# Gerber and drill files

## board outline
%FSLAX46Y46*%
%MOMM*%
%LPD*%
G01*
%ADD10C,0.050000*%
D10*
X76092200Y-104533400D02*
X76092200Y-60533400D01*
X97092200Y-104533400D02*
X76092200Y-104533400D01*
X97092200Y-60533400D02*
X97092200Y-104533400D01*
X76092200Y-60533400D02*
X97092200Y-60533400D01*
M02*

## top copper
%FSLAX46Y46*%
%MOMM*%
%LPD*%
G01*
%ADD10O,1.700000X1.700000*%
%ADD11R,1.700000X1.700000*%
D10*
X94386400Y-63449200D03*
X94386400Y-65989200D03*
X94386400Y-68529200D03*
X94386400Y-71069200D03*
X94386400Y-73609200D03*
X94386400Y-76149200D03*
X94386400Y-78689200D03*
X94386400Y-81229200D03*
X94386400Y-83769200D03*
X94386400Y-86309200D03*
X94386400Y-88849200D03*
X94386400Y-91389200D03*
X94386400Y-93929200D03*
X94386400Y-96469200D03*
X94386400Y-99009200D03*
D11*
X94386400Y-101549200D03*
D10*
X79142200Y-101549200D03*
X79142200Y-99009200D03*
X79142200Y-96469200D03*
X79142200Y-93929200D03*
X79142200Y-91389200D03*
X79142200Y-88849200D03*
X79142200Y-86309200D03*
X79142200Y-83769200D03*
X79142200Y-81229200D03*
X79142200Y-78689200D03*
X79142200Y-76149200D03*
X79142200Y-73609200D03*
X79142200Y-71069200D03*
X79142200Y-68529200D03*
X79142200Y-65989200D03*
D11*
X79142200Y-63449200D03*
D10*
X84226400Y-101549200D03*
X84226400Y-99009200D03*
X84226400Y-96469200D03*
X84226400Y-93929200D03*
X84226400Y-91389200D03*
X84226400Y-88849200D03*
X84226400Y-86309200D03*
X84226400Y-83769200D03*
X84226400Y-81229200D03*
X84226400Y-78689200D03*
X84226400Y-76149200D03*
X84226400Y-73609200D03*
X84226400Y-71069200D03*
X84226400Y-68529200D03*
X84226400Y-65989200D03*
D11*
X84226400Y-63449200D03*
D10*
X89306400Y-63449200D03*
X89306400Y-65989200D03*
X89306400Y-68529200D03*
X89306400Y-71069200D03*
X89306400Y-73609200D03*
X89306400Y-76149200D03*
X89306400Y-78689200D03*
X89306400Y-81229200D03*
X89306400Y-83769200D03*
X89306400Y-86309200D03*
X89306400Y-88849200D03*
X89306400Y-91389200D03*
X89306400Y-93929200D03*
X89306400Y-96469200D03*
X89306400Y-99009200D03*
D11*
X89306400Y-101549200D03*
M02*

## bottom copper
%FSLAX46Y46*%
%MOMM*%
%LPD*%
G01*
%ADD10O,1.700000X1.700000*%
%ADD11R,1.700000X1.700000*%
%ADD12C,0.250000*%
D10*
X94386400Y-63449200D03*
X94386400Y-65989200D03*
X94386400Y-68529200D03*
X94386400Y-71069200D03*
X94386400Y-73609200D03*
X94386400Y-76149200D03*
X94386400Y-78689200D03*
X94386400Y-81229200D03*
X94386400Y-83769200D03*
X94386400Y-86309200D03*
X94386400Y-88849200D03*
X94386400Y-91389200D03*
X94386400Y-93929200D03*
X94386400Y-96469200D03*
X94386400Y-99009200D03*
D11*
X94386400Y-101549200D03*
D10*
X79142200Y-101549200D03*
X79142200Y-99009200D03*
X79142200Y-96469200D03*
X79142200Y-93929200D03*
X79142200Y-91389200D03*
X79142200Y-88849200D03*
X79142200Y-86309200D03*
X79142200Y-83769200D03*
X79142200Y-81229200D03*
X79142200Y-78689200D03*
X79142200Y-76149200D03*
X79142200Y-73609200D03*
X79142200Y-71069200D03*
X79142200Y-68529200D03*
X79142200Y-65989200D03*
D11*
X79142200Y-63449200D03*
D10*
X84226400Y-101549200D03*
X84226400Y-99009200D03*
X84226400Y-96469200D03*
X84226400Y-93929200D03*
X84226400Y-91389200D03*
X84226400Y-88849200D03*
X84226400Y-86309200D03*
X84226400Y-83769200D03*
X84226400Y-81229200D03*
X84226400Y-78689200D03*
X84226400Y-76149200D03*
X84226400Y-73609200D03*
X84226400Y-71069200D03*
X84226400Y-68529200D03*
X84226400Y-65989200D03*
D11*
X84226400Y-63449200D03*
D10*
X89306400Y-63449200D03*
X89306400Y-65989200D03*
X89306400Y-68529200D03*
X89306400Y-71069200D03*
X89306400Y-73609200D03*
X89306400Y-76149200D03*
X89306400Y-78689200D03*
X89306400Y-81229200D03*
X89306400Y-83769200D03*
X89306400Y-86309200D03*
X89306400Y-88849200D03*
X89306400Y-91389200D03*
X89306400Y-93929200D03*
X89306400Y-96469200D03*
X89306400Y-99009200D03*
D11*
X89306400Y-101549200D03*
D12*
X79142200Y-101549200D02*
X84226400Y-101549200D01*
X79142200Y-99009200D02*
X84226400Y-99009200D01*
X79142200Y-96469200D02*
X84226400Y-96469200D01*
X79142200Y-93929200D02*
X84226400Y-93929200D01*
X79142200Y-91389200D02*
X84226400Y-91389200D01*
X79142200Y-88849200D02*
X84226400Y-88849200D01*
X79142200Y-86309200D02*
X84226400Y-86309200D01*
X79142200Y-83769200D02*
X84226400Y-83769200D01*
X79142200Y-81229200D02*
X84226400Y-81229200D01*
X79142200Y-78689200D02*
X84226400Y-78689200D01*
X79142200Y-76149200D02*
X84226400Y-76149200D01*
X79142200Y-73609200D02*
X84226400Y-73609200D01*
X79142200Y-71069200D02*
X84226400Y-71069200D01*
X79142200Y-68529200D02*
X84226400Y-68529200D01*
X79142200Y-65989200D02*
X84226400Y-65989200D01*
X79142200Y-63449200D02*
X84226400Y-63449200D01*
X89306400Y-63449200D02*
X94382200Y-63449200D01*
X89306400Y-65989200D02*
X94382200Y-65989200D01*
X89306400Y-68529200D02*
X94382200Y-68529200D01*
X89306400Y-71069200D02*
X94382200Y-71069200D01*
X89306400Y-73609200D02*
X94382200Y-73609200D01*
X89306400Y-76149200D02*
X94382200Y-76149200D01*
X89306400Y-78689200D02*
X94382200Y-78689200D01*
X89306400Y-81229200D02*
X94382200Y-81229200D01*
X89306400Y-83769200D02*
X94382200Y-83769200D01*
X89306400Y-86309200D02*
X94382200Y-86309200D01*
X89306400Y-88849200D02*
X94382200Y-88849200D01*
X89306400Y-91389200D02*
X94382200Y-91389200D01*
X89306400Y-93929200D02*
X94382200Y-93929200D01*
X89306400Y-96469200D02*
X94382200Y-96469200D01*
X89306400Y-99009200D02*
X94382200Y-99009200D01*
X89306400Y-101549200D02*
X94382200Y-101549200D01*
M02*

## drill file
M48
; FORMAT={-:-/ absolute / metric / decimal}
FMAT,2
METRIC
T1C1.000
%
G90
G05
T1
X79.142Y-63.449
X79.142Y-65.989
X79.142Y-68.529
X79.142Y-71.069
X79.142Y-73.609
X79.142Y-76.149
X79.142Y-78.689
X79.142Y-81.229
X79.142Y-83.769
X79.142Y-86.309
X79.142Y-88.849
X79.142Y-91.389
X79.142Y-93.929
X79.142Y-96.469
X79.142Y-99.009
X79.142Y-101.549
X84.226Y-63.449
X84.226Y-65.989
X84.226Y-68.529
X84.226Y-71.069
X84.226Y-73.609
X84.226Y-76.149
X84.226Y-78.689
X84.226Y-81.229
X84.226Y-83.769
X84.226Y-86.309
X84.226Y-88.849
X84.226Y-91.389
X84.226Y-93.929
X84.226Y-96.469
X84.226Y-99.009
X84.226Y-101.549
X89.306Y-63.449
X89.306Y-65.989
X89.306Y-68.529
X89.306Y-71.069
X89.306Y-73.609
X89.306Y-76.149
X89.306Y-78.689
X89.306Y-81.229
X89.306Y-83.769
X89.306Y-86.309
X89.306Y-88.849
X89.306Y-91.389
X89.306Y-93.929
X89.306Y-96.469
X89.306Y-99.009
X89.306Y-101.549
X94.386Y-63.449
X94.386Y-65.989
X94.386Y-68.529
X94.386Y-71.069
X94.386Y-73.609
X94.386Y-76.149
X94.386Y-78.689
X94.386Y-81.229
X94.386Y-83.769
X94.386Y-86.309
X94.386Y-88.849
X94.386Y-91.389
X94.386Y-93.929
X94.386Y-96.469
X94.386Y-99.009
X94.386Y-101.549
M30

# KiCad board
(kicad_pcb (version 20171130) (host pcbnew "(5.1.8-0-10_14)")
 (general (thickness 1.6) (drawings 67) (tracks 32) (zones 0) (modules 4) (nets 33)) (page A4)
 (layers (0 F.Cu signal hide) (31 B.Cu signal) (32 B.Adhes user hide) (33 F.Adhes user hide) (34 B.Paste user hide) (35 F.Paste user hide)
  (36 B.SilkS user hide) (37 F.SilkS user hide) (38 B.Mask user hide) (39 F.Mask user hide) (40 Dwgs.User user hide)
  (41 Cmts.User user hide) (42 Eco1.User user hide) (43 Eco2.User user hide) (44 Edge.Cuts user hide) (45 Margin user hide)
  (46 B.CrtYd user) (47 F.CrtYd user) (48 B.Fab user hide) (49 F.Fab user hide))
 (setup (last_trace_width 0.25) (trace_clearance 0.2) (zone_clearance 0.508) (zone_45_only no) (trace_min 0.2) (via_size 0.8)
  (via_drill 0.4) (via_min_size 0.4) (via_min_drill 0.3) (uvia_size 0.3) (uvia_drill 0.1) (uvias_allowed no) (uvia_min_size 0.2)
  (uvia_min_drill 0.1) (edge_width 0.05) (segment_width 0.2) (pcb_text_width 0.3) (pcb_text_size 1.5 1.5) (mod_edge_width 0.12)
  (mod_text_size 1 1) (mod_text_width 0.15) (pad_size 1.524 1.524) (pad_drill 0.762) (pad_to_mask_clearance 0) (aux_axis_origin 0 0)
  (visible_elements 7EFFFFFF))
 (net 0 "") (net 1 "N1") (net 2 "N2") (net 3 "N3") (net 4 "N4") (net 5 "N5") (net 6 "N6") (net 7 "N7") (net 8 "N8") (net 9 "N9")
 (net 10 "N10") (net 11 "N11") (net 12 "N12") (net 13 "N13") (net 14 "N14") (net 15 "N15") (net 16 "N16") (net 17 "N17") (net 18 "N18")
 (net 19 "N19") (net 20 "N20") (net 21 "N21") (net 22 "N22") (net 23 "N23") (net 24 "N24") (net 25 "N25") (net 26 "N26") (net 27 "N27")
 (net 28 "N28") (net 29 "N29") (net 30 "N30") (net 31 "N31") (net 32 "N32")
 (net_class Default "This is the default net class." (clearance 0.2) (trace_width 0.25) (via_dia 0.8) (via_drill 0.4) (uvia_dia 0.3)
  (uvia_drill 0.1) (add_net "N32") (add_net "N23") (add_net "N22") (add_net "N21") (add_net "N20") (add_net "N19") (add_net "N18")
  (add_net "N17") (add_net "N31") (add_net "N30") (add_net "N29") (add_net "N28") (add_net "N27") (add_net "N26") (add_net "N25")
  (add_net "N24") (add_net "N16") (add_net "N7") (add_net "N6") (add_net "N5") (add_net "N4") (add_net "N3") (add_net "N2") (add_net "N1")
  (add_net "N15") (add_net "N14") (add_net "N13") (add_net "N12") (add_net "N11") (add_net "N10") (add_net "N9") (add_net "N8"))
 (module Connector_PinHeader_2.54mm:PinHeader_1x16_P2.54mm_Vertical (layer F.Cu) (at 94.3864 101.5492 180)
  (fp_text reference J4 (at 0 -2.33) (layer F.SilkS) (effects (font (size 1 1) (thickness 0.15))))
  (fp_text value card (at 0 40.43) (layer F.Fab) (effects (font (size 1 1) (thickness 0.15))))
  (pad 16 thru_hole oval (at 0 38.1 180) (size 1.7 1.7) (drill 1) (layers *.Cu *.Mask) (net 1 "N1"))
  (pad 15 thru_hole oval (at 0 35.56 180) (size 1.7 1.7) (drill 1) (layers *.Cu *.Mask) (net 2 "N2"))
  (pad 14 thru_hole oval (at 0 33.02 180) (size 1.7 1.7) (drill 1) (layers *.Cu *.Mask) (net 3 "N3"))
  (pad 13 thru_hole oval (at 0 30.48 180) (size 1.7 1.7) (drill 1) (layers *.Cu *.Mask) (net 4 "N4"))
  (pad 12 thru_hole oval (at 0 27.94 180) (size 1.7 1.7) (drill 1) (layers *.Cu *.Mask) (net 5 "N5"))
  (pad 11 thru_hole oval (at 0 25.4 180) (size 1.7 1.7) (drill 1) (layers *.Cu *.Mask) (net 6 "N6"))
  (pad 10 thru_hole oval (at 0 22.86 180) (size 1.7 1.7) (drill 1) (layers *.Cu *.Mask) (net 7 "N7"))
  (pad 9 thru_hole oval (at 0 20.32 180) (size 1.7 1.7) (drill 1) (layers *.Cu *.Mask) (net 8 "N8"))
  (pad 8 thru_hole oval (at 0 17.78 180) (size 1.7 1.7) (drill 1) (layers *.Cu *.Mask) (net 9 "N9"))
  (pad 7 thru_hole oval (at 0 15.24 180) (size 1.7 1.7) (drill 1) (layers *.Cu *.Mask) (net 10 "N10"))
  (pad 6 thru_hole oval (at 0 12.7 180) (size 1.7 1.7) (drill 1) (layers *.Cu *.Mask) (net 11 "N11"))
  (pad 5 thru_hole oval (at 0 10.16 180) (size 1.7 1.7) (drill 1) (layers *.Cu *.Mask) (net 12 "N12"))
  (pad 4 thru_hole oval (at 0 7.62 180) (size 1.7 1.7) (drill 1) (layers *.Cu *.Mask) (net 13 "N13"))
  (pad 3 thru_hole oval (at 0 5.08 180) (size 1.7 1.7) (drill 1) (layers *.Cu *.Mask) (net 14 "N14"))
  (pad 2 thru_hole oval (at 0 2.54 180) (size 1.7 1.7) (drill 1) (layers *.Cu *.Mask) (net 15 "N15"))
  (pad 1 thru_hole rect (at 0 0 180) (size 1.7 1.7) (drill 1) (layers *.Cu *.Mask) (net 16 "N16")))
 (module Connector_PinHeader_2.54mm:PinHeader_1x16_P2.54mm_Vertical (layer F.Cu) (at 79.1422 63.4492)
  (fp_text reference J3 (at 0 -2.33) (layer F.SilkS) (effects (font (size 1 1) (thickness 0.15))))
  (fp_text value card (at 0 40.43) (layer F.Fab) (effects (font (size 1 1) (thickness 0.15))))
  (pad 16 thru_hole oval (at 0 38.1) (size 1.7 1.7) (drill 1) (layers *.Cu *.Mask) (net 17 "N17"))
  (pad 15 thru_hole oval (at 0 35.56) (size 1.7 1.7) (drill 1) (layers *.Cu *.Mask) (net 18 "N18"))
  (pad 14 thru_hole oval (at 0 33.02) (size 1.7 1.7) (drill 1) (layers *.Cu *.Mask) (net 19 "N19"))
  (pad 13 thru_hole oval (at 0 30.48) (size 1.7 1.7) (drill 1) (layers *.Cu *.Mask) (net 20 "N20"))
  (pad 12 thru_hole oval (at 0 27.94) (size 1.7 1.7) (drill 1) (layers *.Cu *.Mask) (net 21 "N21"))
  (pad 11 thru_hole oval (at 0 25.4) (size 1.7 1.7) (drill 1) (layers *.Cu *.Mask) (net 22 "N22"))
  (pad 10 thru_hole oval (at 0 22.86) (size 1.7 1.7) (drill 1) (layers *.Cu *.Mask) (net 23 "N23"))
  (pad 9 thru_hole oval (at 0 20.32) (size 1.7 1.7) (drill 1) (layers *.Cu *.Mask) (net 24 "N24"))
  (pad 8 thru_hole oval (at 0 17.78) (size 1.7 1.7) (drill 1) (layers *.Cu *.Mask) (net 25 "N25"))
  (pad 7 thru_hole oval (at 0 15.24) (size 1.7 1.7) (drill 1) (layers *.Cu *.Mask) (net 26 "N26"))
  (pad 6 thru_hole oval (at 0 12.7) (size 1.7 1.7) (drill 1) (layers *.Cu *.Mask) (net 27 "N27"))
  (pad 5 thru_hole oval (at 0 10.16) (size 1.7 1.7) (drill 1) (layers *.Cu *.Mask) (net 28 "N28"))
  (pad 4 thru_hole oval (at 0 7.62) (size 1.7 1.7) (drill 1) (layers *.Cu *.Mask) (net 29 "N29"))
  (pad 3 thru_hole oval (at 0 5.08) (size 1.7 1.7) (drill 1) (layers *.Cu *.Mask) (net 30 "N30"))
  (pad 2 thru_hole oval (at 0 2.54) (size 1.7 1.7) (drill 1) (layers *.Cu *.Mask) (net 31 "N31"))
  (pad 1 thru_hole rect (at 0 0) (size 1.7 1.7) (drill 1) (layers *.Cu *.Mask) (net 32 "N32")))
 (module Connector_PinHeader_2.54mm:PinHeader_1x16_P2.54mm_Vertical (layer B.Cu) (at 84.2264 63.4492 180)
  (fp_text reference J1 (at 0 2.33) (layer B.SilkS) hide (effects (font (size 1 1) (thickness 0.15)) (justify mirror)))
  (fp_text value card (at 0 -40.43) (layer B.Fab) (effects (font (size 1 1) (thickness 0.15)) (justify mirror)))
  (pad 16 thru_hole oval (at 0 -38.1 180) (size 1.7 1.7) (drill 1) (layers *.Cu *.Mask) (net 17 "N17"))
  (pad 15 thru_hole oval (at 0 -35.56 180) (size 1.7 1.7) (drill 1) (layers *.Cu *.Mask) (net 18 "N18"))
  (pad 14 thru_hole oval (at 0 -33.02 180) (size 1.7 1.7) (drill 1) (layers *.Cu *.Mask) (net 19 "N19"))
  (pad 13 thru_hole oval (at 0 -30.48 180) (size 1.7 1.7) (drill 1) (layers *.Cu *.Mask) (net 20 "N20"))
  (pad 12 thru_hole oval (at 0 -27.94 180) (size 1.7 1.7) (drill 1) (layers *.Cu *.Mask) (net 21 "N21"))
  (pad 11 thru_hole oval (at 0 -25.4 180) (size 1.7 1.7) (drill 1) (layers *.Cu *.Mask) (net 22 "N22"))
  (pad 10 thru_hole oval (at 0 -22.86 180) (size 1.7 1.7) (drill 1) (layers *.Cu *.Mask) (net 23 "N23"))
  (pad 9 thru_hole oval (at 0 -20.32 180) (size 1.7 1.7) (drill 1) (layers *.Cu *.Mask) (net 24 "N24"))
  (pad 8 thru_hole oval (at 0 -17.78 180) (size 1.7 1.7) (drill 1) (layers *.Cu *.Mask) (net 25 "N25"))
  (pad 7 thru_hole oval (at 0 -15.24 180) (size 1.7 1.7) (drill 1) (layers *.Cu *.Mask) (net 26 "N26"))
  (pad 6 thru_hole oval (at 0 -12.7 180) (size 1.7 1.7) (drill 1) (layers *.Cu *.Mask) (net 27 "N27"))
  (pad 5 thru_hole oval (at 0 -10.16 180) (size 1.7 1.7) (drill 1) (layers *.Cu *.Mask) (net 28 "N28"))
  (pad 4 thru_hole oval (at 0 -7.62 180) (size 1.7 1.7) (drill 1) (layers *.Cu *.Mask) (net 29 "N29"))
  (pad 3 thru_hole oval (at 0 -5.08 180) (size 1.7 1.7) (drill 1) (layers *.Cu *.Mask) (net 30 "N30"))
  (pad 2 thru_hole oval (at 0 -2.54 180) (size 1.7 1.7) (drill 1) (layers *.Cu *.Mask) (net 31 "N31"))
  (pad 1 thru_hole rect (at 0 0 180) (size 1.7 1.7) (drill 1) (layers *.Cu *.Mask) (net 32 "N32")))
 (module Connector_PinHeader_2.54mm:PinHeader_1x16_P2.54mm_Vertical (layer B.Cu) (at 89.3064 101.5492)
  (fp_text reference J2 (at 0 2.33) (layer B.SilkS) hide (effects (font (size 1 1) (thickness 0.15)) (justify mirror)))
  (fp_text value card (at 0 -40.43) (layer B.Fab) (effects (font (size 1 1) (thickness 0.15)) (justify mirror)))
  (pad 16 thru_hole oval (at 0 -38.1) (size 1.7 1.7) (drill 1) (layers *.Cu *.Mask) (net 1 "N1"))
  (pad 15 thru_hole oval (at 0 -35.56) (size 1.7 1.7) (drill 1) (layers *.Cu *.Mask) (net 2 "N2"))
  (pad 14 thru_hole oval (at 0 -33.02) (size 1.7 1.7) (drill 1) (layers *.Cu *.Mask) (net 3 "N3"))
  (pad 13 thru_hole oval (at 0 -30.48) (size 1.7 1.7) (drill 1) (layers *.Cu *.Mask) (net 4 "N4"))
  (pad 12 thru_hole oval (at 0 -27.94) (size 1.7 1.7) (drill 1) (layers *.Cu *.Mask) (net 5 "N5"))
  (pad 11 thru_hole oval (at 0 -25.4) (size 1.7 1.7) (drill 1) (layers *.Cu *.Mask) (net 6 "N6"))
  (pad 10 thru_hole oval (at 0 -22.86) (size 1.7 1.7) (drill 1) (layers *.Cu *.Mask) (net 7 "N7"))
  (pad 9 thru_hole oval (at 0 -20.32) (size 1.7 1.7) (drill 1) (layers *.Cu *.Mask) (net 8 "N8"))
  (pad 8 thru_hole oval (at 0 -17.78) (size 1.7 1.7) (drill 1) (layers *.Cu *.Mask) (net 9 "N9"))
  (pad 7 thru_hole oval (at 0 -15.24) (size 1.7 1.7) (drill 1) (layers *.Cu *.Mask) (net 10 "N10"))
  (pad 6 thru_hole oval (at 0 -12.7) (size 1.7 1.7) (drill 1) (layers *.Cu *.Mask) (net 11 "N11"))
  (pad 5 thru_hole oval (at 0 -10.16) (size 1.7 1.7) (drill 1) (layers *.Cu *.Mask) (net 12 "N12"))
  (pad 4 thru_hole oval (at 0 -7.62) (size 1.7 1.7) (drill 1) (layers *.Cu *.Mask) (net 13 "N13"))
  (pad 3 thru_hole oval (at 0 -5.08) (size 1.7 1.7) (drill 1) (layers *.Cu *.Mask) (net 14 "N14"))
  (pad 2 thru_hole oval (at 0 -2.54) (size 1.7 1.7) (drill 1) (layers *.Cu *.Mask) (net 15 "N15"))
  (pad 1 thru_hole rect (at 0 0) (size 1.7 1.7) (drill 1) (layers *.Cu *.Mask) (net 16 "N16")))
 (gr_line (start 76.0922 104.5334) (end 76.0922 60.5334) (layer Edge.Cuts) (width 0.05))
 (gr_line (start 97.0922 104.5334) (end 76.0922 104.5334) (layer Edge.Cuts) (width 0.05))
 (gr_line (start 97.0922 60.5334) (end 97.0922 104.5334) (layer Edge.Cuts) (width 0.05))
 (gr_line (start 76.0922 60.5334) (end 97.0922 60.5334) (layer Edge.Cuts) (width 0.05))
 (segment (start 79.1422 101.5492) (end 84.2264 101.5492) (width 0.25) (layer B.Cu) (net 17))
 (segment (start 79.1422 99.0092) (end 84.2264 99.0092) (width 0.25) (layer B.Cu) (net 18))
 (segment (start 79.1422 96.4692) (end 84.2264 96.4692) (width 0.25) (layer B.Cu) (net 19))
 (segment (start 79.1422 93.9292) (end 84.2264 93.9292) (width 0.25) (layer B.Cu) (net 20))
 (segment (start 79.1422 91.3892) (end 84.2264 91.3892) (width 0.25) (layer B.Cu) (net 21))
 (segment (start 79.1422 88.8492) (end 84.2264 88.8492) (width 0.25) (layer B.Cu) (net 22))
 (segment (start 79.1422 86.3092) (end 84.2264 86.3092) (width 0.25) (layer B.Cu) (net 23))
 (segment (start 79.1422 83.7692) (end 84.2264 83.7692) (width 0.25) (layer B.Cu) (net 24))
 (segment (start 79.1422 81.2292) (end 84.2264 81.2292) (width 0.25) (layer B.Cu) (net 25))
 (segment (start 79.1422 78.6892) (end 84.2264 78.6892) (width 0.25) (layer B.Cu) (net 26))
 (segment (start 79.1422 76.1492) (end 84.2264 76.1492) (width 0.25) (layer B.Cu) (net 27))
 (segment (start 79.1422 73.6092) (end 84.2264 73.6092) (width 0.25) (layer B.Cu) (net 28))
 (segment (start 79.1422 71.0692) (end 84.2264 71.0692) (width 0.25) (layer B.Cu) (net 29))
 (segment (start 79.1422 68.5292) (end 84.2264 68.5292) (width 0.25) (layer B.Cu) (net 30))
 (segment (start 79.1422 65.9892) (end 84.2264 65.9892) (width 0.25) (layer B.Cu) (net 31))
 (segment (start 79.1422 63.4492) (end 84.2264 63.4492) (width 0.25) (layer B.Cu) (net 32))
 (segment (start 89.3064 63.4492) (end 94.3822 63.4492) (width 0.25) (layer B.Cu) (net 1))
 (segment (start 89.3064 65.9892) (end 94.3822 65.9892) (width 0.25) (layer B.Cu) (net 2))
 (segment (start 89.3064 68.5292) (end 94.3822 68.5292) (width 0.25) (layer B.Cu) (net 3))
 (segment (start 89.3064 71.0692) (end 94.3822 71.0692) (width 0.25) (layer B.Cu) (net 4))
 (segment (start 89.3064 73.6092) (end 94.3822 73.6092) (width 0.25) (layer B.Cu) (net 5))
 (segment (start 89.3064 76.1492) (end 94.3822 76.1492) (width 0.25) (layer B.Cu) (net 6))
 (segment (start 89.3064 78.6892) (end 94.3822 78.6892) (width 0.25) (layer B.Cu) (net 7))
 (segment (start 89.3064 81.2292) (end 94.3822 81.2292) (width 0.25) (layer B.Cu) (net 8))
 (segment (start 89.3064 83.7692) (end 94.3822 83.7692) (width 0.25) (layer B.Cu) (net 9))
 (segment (start 89.3064 86.3092) (end 94.3822 86.3092) (width 0.25) (layer B.Cu) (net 10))
 (segment (start 89.3064 88.8492) (end 94.3822 88.8492) (width 0.25) (layer B.Cu) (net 11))
 (segment (start 89.3064 91.3892) (end 94.3822 91.3892) (width 0.25) (layer B.Cu) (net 12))
 (segment (start 89.3064 93.9292) (end 94.3822 93.9292) (width 0.25) (layer B.Cu) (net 13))
 (segment (start 89.3064 96.4692) (end 94.3822 96.4692) (width 0.25) (layer B.Cu) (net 14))
 (segment (start 89.3064 99.0092) (end 94.3822 99.0092) (width 0.25) (layer B.Cu) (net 15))
 (segment (start 89.3064 101.5492) (end 94.3822 101.5492) (width 0.25) (layer B.Cu) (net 16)))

